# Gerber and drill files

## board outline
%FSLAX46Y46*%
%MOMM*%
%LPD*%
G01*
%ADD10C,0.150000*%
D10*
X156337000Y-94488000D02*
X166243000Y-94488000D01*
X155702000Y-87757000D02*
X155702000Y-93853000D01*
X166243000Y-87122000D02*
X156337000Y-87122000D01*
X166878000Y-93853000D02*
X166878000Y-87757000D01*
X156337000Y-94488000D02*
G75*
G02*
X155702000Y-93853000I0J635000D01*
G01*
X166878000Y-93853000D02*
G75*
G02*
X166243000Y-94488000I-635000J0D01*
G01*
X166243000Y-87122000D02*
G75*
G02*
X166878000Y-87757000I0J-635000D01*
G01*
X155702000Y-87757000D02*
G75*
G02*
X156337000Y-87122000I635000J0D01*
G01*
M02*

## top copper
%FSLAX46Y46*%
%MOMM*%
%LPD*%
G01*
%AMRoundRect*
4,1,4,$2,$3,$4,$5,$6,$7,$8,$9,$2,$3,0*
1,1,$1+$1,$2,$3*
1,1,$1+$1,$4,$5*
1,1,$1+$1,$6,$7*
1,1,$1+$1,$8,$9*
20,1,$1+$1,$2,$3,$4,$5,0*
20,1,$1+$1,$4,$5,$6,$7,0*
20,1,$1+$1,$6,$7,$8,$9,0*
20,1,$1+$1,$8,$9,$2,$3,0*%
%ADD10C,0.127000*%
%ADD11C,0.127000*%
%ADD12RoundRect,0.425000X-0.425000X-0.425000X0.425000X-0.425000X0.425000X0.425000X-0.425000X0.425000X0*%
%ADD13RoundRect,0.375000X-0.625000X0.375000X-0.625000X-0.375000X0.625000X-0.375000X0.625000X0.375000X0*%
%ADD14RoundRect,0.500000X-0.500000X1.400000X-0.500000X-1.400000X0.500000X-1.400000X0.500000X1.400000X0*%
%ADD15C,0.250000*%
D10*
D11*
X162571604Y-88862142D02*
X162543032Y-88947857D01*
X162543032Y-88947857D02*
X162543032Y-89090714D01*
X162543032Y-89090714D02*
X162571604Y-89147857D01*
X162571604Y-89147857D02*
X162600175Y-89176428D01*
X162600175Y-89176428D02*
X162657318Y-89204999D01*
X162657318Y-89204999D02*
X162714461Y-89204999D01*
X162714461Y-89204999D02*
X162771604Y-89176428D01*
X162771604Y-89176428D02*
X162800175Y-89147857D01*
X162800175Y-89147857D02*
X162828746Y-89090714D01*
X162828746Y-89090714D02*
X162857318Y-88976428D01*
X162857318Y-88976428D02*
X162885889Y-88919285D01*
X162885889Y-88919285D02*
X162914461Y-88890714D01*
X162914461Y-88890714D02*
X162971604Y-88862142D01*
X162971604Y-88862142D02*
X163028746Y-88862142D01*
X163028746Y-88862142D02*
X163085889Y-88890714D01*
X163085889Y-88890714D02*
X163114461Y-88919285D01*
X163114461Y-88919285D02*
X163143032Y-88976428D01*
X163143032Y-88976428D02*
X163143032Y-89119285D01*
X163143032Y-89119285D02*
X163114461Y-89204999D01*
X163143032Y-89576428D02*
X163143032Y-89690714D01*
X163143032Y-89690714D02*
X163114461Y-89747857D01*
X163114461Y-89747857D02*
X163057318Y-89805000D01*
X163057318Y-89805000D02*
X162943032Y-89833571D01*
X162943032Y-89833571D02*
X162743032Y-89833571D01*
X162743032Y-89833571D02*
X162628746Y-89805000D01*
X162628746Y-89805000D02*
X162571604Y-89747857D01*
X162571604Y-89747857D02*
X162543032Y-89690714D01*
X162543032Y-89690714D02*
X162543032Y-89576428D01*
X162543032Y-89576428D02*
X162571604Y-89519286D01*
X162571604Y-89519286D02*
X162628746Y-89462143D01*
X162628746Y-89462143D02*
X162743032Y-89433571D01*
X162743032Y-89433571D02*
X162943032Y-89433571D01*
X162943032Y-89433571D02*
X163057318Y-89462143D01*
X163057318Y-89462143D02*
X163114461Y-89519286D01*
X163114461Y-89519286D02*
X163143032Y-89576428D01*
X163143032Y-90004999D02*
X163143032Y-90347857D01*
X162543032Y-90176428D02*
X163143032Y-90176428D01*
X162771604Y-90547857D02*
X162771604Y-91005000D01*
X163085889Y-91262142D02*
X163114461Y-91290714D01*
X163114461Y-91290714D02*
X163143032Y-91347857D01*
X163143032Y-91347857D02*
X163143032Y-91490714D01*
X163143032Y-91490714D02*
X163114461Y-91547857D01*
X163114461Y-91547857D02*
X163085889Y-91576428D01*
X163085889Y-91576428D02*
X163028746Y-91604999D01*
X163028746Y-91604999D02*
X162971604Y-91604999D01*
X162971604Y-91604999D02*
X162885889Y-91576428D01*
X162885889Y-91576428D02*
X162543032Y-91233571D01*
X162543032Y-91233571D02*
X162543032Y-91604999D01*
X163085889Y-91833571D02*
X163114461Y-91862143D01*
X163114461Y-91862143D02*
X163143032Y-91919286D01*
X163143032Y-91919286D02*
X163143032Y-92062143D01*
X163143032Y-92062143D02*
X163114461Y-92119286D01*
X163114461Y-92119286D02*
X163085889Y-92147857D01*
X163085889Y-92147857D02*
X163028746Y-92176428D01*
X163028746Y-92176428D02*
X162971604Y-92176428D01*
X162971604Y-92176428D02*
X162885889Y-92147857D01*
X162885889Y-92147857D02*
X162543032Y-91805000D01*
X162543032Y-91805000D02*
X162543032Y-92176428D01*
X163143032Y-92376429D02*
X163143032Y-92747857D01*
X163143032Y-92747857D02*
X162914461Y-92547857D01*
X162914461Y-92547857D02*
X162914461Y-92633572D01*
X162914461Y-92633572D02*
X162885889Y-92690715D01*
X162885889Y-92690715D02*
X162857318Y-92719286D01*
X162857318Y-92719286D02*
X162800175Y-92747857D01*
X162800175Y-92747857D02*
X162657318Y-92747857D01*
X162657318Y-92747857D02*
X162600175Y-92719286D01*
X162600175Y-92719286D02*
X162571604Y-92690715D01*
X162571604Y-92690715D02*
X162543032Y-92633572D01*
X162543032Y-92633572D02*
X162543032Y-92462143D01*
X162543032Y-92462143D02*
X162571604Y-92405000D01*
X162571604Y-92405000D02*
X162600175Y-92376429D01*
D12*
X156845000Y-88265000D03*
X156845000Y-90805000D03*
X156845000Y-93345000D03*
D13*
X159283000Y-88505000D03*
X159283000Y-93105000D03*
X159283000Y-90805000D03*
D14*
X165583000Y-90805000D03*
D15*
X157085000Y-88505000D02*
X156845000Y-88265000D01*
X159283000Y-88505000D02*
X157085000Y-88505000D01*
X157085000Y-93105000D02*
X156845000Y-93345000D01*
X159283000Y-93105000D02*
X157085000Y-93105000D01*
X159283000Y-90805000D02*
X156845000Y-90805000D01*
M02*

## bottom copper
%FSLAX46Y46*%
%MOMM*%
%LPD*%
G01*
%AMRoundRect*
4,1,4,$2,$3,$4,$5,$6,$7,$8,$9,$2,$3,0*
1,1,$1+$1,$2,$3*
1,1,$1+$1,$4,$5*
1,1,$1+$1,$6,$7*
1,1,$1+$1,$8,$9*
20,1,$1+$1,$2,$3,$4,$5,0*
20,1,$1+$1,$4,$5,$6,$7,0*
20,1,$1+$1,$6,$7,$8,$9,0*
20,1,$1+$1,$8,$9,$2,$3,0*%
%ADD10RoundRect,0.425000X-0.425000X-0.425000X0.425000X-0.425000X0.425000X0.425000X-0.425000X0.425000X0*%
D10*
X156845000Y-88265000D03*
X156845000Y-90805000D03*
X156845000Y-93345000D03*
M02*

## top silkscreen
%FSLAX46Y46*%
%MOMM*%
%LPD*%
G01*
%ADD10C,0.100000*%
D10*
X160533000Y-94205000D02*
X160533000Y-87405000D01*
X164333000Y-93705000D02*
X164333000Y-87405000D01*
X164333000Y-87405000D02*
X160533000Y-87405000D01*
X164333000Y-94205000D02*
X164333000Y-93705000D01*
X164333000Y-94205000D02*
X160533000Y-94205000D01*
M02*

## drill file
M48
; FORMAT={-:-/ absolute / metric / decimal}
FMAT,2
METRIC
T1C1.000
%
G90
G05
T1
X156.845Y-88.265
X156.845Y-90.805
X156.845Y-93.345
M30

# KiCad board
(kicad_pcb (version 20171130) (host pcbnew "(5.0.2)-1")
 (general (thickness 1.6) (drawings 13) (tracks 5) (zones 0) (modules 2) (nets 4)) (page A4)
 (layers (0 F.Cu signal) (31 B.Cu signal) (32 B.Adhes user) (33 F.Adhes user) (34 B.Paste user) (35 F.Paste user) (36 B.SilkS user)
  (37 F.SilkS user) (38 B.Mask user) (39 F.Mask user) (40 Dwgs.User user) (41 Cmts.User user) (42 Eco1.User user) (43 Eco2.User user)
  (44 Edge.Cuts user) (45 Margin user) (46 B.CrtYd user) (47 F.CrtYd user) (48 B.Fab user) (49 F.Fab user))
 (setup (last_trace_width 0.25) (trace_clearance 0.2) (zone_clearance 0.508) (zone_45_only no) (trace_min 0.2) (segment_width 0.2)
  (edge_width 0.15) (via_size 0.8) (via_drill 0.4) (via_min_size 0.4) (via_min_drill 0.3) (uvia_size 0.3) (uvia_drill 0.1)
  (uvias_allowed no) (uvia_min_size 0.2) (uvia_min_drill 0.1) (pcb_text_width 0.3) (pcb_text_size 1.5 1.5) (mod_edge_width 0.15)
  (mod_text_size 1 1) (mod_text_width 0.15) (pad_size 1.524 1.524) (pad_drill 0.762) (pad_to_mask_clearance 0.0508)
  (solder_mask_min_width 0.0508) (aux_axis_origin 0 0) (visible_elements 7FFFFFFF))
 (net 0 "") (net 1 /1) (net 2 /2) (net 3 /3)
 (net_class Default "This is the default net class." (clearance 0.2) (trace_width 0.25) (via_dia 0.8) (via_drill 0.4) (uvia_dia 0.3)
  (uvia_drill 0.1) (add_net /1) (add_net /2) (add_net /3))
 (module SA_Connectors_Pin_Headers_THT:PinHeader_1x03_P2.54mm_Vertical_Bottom (layer F.Cu) (at 156.845 88.265)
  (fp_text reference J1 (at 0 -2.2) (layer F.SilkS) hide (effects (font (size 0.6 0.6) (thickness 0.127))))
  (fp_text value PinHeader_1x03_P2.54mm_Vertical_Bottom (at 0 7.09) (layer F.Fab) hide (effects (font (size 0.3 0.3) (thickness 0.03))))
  (pad 1 thru_hole roundrect (at 0 0) (size 1.7 1.7) (drill 1) (layers *.Cu *.Mask) (roundrect_rratio 0.25) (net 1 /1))
  (pad 2 thru_hole roundrect (at 0 2.54) (size 1.7 1.7) (drill 1) (layers *.Cu *.Mask) (roundrect_rratio 0.25) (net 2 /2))
  (pad 3 thru_hole roundrect (at 0 5.08) (size 1.7 1.7) (drill 1) (layers *.Cu *.Mask) (roundrect_rratio 0.25) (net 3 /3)))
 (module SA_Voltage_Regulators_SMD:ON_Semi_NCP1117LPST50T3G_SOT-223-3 (layer F.Cu) (at 162.433 90.805 270)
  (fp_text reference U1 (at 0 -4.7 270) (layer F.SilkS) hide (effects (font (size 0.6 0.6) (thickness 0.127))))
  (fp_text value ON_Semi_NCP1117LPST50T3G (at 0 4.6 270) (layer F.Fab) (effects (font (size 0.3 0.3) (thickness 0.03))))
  (fp_line (start 3.4 1.9) (end -3.4 1.9) (layer F.SilkS) (width 0.1))
  (fp_line (start 2.9 -1.9) (end -3.4 -1.9) (layer F.SilkS) (width 0.1))
  (fp_line (start -3.4 -1.9) (end -3.4 1.9) (layer F.SilkS) (width 0.1))
  (fp_line (start 3.4 -1.9) (end 2.9 -1.9) (layer F.SilkS) (width 0.1))
  (fp_line (start 3.4 -1.9) (end 3.4 1.9) (layer F.SilkS) (width 0.1))
  (pad 1 smd roundrect (at -2.3 3.15 270) (size 1.5 2) (layers F.Cu F.Paste F.Mask) (roundrect_rratio 0.25) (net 1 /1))
  (pad 3 smd roundrect (at 2.3 3.15 270) (size 1.5 2) (layers F.Cu F.Paste F.Mask) (roundrect_rratio 0.25) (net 3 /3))
  (pad 2 smd roundrect (at 0 3.15 270) (size 1.5 2) (layers F.Cu F.Paste F.Mask) (roundrect_rratio 0.25) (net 2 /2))
  (pad 2 smd roundrect (at 0 -3.15 270) (size 3.8 2) (layers F.Cu F.Paste F.Mask) (roundrect_rratio 0.25) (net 2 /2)))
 (gr_line (start 156.337 94.488) (end 166.243 94.488) (layer Edge.Cuts) (width 0.15))
 (gr_line (start 155.702 87.757) (end 155.702 93.853) (layer Edge.Cuts) (width 0.15))
 (gr_line (start 166.243 87.122) (end 156.337 87.122) (layer Edge.Cuts) (width 0.15))
 (gr_line (start 166.878 93.853) (end 166.878 87.757) (layer Edge.Cuts) (width 0.15))
 (gr_arc (start 156.337 93.853) (end 155.702 93.853) (angle -90) (layer Edge.Cuts) (width 0.15))
 (gr_arc (start 166.243 93.853) (end 166.243 94.488) (angle -90) (layer Edge.Cuts) (width 0.15))
 (gr_arc (start 166.243 87.757) (end 166.878 87.757) (angle -90) (layer Edge.Cuts) (width 0.15))
 (gr_arc (start 156.337 87.757) (end 156.337 87.122) (angle -90) (layer Edge.Cuts) (width 0.15))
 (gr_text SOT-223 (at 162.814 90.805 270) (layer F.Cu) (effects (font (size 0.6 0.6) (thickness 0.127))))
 (segment (start 157.085 88.505) (end 156.845 88.265) (width 0.25) (layer F.Cu) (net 1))
 (segment (start 159.283 88.505) (end 157.085 88.505) (width 0.25) (layer F.Cu) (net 1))
 (segment (start 157.085 93.105) (end 156.845 93.345) (width 0.25) (layer F.Cu) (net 3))
 (segment (start 159.283 93.105) (end 157.085 93.105) (width 0.25) (layer F.Cu) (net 3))
 (segment (start 159.283 90.805) (end 156.845 90.805) (width 0.25) (layer F.Cu) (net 2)))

